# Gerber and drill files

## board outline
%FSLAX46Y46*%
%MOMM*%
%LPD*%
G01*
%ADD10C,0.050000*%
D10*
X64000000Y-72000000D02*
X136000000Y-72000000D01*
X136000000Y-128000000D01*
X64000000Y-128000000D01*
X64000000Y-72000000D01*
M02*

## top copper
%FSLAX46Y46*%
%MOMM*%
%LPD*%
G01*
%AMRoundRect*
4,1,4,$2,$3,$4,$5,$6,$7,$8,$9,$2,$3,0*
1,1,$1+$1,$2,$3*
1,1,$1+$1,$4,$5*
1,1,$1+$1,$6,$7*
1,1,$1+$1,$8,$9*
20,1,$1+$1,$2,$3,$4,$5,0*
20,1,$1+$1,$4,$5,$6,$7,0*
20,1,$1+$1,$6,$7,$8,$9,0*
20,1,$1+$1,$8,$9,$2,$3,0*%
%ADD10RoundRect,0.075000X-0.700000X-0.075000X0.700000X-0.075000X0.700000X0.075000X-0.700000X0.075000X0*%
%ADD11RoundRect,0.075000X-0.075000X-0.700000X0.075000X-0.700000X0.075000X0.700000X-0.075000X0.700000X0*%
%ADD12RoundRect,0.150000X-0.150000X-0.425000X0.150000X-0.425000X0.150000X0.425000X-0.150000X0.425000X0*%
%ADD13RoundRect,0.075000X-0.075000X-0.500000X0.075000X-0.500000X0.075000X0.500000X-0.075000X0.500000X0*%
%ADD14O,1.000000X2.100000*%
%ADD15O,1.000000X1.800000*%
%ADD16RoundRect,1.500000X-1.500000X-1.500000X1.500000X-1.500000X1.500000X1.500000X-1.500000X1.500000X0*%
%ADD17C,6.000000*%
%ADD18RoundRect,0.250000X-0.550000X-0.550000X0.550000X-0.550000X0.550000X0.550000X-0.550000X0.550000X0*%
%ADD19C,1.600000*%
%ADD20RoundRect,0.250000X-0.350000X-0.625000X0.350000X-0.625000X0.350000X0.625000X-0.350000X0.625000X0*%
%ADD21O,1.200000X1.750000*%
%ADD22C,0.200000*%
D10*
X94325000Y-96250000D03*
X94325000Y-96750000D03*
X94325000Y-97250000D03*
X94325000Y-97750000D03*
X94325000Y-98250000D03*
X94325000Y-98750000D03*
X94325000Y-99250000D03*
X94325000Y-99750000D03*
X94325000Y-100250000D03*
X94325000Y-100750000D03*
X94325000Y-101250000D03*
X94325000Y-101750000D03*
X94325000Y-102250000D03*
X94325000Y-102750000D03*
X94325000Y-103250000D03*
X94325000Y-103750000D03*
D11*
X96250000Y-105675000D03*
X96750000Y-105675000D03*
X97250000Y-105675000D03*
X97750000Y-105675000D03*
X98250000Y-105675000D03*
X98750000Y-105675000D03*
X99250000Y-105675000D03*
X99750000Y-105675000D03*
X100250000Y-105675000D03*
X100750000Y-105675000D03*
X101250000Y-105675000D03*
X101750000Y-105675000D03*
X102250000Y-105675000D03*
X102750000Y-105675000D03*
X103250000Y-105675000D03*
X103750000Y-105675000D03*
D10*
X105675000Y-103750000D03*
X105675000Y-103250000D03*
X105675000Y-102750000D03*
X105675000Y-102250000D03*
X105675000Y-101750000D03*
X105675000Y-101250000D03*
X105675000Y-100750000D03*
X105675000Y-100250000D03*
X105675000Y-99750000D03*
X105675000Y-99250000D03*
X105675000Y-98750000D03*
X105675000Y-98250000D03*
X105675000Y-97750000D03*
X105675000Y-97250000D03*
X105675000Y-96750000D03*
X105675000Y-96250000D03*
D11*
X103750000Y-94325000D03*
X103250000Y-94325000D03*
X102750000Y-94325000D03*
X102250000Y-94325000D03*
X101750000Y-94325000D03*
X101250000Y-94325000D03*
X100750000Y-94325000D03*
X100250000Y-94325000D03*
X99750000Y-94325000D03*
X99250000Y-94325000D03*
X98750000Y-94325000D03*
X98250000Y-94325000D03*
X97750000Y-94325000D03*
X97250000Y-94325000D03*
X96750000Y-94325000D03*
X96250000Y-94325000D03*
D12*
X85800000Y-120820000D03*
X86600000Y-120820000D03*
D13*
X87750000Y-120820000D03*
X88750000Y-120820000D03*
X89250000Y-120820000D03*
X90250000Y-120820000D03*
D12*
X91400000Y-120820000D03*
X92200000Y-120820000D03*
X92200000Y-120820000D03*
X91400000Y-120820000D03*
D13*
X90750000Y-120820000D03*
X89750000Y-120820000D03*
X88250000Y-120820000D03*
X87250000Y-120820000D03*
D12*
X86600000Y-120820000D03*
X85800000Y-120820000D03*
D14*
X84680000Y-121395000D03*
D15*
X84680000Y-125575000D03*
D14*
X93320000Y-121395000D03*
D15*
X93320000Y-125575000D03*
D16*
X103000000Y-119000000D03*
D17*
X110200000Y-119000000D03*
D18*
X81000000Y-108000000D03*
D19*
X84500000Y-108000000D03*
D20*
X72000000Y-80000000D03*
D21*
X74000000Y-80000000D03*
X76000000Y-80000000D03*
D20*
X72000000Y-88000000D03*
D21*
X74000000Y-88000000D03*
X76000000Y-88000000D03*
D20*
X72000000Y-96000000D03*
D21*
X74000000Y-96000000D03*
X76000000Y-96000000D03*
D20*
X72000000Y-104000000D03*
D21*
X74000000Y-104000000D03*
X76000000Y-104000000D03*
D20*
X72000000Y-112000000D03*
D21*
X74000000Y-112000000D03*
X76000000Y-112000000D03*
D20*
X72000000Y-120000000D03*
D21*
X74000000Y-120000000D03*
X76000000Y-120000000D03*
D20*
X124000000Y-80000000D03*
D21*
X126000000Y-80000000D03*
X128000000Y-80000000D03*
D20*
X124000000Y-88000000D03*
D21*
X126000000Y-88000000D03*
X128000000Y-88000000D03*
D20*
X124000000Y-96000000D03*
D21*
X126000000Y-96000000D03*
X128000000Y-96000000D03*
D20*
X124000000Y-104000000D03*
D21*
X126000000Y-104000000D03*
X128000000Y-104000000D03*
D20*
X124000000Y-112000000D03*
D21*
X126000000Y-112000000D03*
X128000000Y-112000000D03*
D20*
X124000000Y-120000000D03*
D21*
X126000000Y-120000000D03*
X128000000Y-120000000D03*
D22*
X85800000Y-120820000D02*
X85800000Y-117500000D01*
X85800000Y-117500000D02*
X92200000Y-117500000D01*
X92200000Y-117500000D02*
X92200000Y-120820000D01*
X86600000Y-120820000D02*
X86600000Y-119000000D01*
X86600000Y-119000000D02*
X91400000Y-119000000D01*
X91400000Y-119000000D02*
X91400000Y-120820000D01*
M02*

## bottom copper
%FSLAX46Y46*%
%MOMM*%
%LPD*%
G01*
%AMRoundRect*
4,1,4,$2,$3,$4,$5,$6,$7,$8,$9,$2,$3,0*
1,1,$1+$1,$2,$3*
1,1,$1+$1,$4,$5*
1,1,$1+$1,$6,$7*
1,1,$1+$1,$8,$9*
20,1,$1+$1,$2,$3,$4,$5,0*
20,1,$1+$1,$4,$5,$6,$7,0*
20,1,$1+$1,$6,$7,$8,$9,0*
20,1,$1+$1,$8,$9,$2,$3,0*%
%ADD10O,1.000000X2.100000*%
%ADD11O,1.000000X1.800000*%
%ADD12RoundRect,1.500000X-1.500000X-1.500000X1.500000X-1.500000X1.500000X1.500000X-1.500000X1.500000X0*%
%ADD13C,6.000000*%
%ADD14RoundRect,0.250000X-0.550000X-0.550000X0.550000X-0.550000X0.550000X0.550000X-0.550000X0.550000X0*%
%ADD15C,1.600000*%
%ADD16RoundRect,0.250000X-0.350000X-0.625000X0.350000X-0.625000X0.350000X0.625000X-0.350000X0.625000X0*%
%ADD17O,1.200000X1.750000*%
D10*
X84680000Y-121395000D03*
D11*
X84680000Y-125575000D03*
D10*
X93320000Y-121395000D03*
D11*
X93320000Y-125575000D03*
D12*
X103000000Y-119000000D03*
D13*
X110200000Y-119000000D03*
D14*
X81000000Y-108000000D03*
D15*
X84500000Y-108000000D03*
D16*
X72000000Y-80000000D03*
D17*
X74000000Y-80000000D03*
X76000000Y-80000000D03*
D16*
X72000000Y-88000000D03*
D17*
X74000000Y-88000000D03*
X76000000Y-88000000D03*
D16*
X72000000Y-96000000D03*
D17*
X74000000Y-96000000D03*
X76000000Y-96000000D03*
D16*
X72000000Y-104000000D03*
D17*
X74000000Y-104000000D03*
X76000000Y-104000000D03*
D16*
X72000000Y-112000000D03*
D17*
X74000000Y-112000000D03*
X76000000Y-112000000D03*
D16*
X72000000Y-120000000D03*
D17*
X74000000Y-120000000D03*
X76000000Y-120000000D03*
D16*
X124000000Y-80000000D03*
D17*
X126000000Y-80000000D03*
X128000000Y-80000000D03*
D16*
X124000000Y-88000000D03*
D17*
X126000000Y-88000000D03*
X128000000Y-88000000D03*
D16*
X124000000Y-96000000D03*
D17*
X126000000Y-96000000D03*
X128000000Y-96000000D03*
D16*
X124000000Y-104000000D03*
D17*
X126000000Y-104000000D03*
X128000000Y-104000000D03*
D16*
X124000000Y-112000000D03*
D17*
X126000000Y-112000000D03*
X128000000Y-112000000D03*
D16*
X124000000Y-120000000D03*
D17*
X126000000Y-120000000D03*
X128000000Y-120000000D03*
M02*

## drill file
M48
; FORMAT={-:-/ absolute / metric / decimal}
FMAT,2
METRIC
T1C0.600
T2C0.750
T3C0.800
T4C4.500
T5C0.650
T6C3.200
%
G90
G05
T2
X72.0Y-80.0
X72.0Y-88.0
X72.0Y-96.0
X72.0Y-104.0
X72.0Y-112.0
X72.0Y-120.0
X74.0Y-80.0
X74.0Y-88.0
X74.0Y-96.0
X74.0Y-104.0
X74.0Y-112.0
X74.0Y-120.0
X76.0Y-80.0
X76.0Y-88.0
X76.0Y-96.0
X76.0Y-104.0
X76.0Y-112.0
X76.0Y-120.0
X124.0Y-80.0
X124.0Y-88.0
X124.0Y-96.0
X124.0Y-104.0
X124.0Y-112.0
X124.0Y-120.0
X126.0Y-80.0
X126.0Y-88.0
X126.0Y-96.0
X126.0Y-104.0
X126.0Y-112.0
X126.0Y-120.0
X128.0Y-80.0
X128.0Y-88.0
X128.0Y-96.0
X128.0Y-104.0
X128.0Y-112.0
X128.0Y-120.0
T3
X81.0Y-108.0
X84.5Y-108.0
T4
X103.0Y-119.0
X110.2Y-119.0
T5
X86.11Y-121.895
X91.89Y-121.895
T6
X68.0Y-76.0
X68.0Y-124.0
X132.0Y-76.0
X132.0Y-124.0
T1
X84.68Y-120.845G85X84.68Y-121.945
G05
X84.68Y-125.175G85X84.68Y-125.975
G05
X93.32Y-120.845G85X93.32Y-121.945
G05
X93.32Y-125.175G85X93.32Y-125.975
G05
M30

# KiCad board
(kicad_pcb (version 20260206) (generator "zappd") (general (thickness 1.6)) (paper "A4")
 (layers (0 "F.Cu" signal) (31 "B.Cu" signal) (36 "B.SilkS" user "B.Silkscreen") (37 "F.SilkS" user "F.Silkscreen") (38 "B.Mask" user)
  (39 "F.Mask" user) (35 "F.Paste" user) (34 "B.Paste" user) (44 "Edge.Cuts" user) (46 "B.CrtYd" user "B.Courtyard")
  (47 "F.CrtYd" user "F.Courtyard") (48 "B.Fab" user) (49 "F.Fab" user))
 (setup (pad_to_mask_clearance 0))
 (gr_rect (start 64.0 72.0) (end 136.0 128.0) (stroke (width 0.05) (type default)) (fill none) (layer "Edge.Cuts"))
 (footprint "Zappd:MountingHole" (layer "F.Cu") (at 68.0 76.0)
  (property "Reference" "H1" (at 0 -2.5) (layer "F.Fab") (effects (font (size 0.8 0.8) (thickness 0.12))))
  (pad "" np_thru_hole circle (at 0 0) (size 3.2 3.2) (drill 3.2) (layers "*.Cu" "*.Mask")))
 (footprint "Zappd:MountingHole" (layer "F.Cu") (at 132.0 76.0)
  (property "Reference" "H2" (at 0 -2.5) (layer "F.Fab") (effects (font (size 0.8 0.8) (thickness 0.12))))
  (pad "" np_thru_hole circle (at 0 0) (size 3.2 3.2) (drill 3.2) (layers "*.Cu" "*.Mask")))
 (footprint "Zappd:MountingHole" (layer "F.Cu") (at 132.0 124.0)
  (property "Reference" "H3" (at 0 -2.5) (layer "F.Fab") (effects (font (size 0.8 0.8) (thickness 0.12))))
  (pad "" np_thru_hole circle (at 0 0) (size 3.2 3.2) (drill 3.2) (layers "*.Cu" "*.Mask")))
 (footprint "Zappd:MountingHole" (layer "F.Cu") (at 68.0 124.0)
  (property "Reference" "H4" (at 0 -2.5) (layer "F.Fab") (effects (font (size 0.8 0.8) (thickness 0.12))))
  (pad "" np_thru_hole circle (at 0 0) (size 3.2 3.2) (drill 3.2) (layers "*.Cu" "*.Mask")))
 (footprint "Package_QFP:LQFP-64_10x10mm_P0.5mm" (layer "F.Cu") (at 100 100)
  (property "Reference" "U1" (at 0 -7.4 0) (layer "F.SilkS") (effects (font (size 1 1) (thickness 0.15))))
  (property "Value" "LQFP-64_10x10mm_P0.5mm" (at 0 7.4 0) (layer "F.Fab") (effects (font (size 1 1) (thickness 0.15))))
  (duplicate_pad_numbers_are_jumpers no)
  (pad "1" smd roundrect (at -5.675 -3.75) (size 1.55 0.3) (layers "F.Cu" "F.Mask" "F.Paste") (roundrect_rratio 0.25))
  (pad "2" smd roundrect (at -5.675 -3.25) (size 1.55 0.3) (layers "F.Cu" "F.Mask" "F.Paste") (roundrect_rratio 0.25))
  (pad "3" smd roundrect (at -5.675 -2.75) (size 1.55 0.3) (layers "F.Cu" "F.Mask" "F.Paste") (roundrect_rratio 0.25))
  (pad "4" smd roundrect (at -5.675 -2.25) (size 1.55 0.3) (layers "F.Cu" "F.Mask" "F.Paste") (roundrect_rratio 0.25))
  (pad "5" smd roundrect (at -5.675 -1.75) (size 1.55 0.3) (layers "F.Cu" "F.Mask" "F.Paste") (roundrect_rratio 0.25))
  (pad "6" smd roundrect (at -5.675 -1.25) (size 1.55 0.3) (layers "F.Cu" "F.Mask" "F.Paste") (roundrect_rratio 0.25))
  (pad "7" smd roundrect (at -5.675 -0.75) (size 1.55 0.3) (layers "F.Cu" "F.Mask" "F.Paste") (roundrect_rratio 0.25))
  (pad "8" smd roundrect (at -5.675 -0.25) (size 1.55 0.3) (layers "F.Cu" "F.Mask" "F.Paste") (roundrect_rratio 0.25))
  (pad "9" smd roundrect (at -5.675 0.25) (size 1.55 0.3) (layers "F.Cu" "F.Mask" "F.Paste") (roundrect_rratio 0.25))
  (pad "10" smd roundrect (at -5.675 0.75) (size 1.55 0.3) (layers "F.Cu" "F.Mask" "F.Paste") (roundrect_rratio 0.25))
  (pad "11" smd roundrect (at -5.675 1.25) (size 1.55 0.3) (layers "F.Cu" "F.Mask" "F.Paste") (roundrect_rratio 0.25))
  (pad "12" smd roundrect (at -5.675 1.75) (size 1.55 0.3) (layers "F.Cu" "F.Mask" "F.Paste") (roundrect_rratio 0.25))
  (pad "13" smd roundrect (at -5.675 2.25) (size 1.55 0.3) (layers "F.Cu" "F.Mask" "F.Paste") (roundrect_rratio 0.25))
  (pad "14" smd roundrect (at -5.675 2.75) (size 1.55 0.3) (layers "F.Cu" "F.Mask" "F.Paste") (roundrect_rratio 0.25))
  (pad "15" smd roundrect (at -5.675 3.25) (size 1.55 0.3) (layers "F.Cu" "F.Mask" "F.Paste") (roundrect_rratio 0.25))
  (pad "16" smd roundrect (at -5.675 3.75) (size 1.55 0.3) (layers "F.Cu" "F.Mask" "F.Paste") (roundrect_rratio 0.25))
  (pad "17" smd roundrect (at -3.75 5.675) (size 0.3 1.55) (layers "F.Cu" "F.Mask" "F.Paste") (roundrect_rratio 0.25))
  (pad "18" smd roundrect (at -3.25 5.675) (size 0.3 1.55) (layers "F.Cu" "F.Mask" "F.Paste") (roundrect_rratio 0.25))
  (pad "19" smd roundrect (at -2.75 5.675) (size 0.3 1.55) (layers "F.Cu" "F.Mask" "F.Paste") (roundrect_rratio 0.25))
  (pad "20" smd roundrect (at -2.25 5.675) (size 0.3 1.55) (layers "F.Cu" "F.Mask" "F.Paste") (roundrect_rratio 0.25))
  (pad "21" smd roundrect (at -1.75 5.675) (size 0.3 1.55) (layers "F.Cu" "F.Mask" "F.Paste") (roundrect_rratio 0.25))
  (pad "22" smd roundrect (at -1.25 5.675) (size 0.3 1.55) (layers "F.Cu" "F.Mask" "F.Paste") (roundrect_rratio 0.25))
  (pad "23" smd roundrect (at -0.75 5.675) (size 0.3 1.55) (layers "F.Cu" "F.Mask" "F.Paste") (roundrect_rratio 0.25))
  (pad "24" smd roundrect (at -0.25 5.675) (size 0.3 1.55) (layers "F.Cu" "F.Mask" "F.Paste") (roundrect_rratio 0.25))
  (pad "25" smd roundrect (at 0.25 5.675) (size 0.3 1.55) (layers "F.Cu" "F.Mask" "F.Paste") (roundrect_rratio 0.25))
  (pad "26" smd roundrect (at 0.75 5.675) (size 0.3 1.55) (layers "F.Cu" "F.Mask" "F.Paste") (roundrect_rratio 0.25))
  (pad "27" smd roundrect (at 1.25 5.675) (size 0.3 1.55) (layers "F.Cu" "F.Mask" "F.Paste") (roundrect_rratio 0.25))
  (pad "28" smd roundrect (at 1.75 5.675) (size 0.3 1.55) (layers "F.Cu" "F.Mask" "F.Paste") (roundrect_rratio 0.25))
  (pad "29" smd roundrect (at 2.25 5.675) (size 0.3 1.55) (layers "F.Cu" "F.Mask" "F.Paste") (roundrect_rratio 0.25))
  (pad "30" smd roundrect (at 2.75 5.675) (size 0.3 1.55) (layers "F.Cu" "F.Mask" "F.Paste") (roundrect_rratio 0.25))
  (pad "31" smd roundrect (at 3.25 5.675) (size 0.3 1.55) (layers "F.Cu" "F.Mask" "F.Paste") (roundrect_rratio 0.25))
  (pad "32" smd roundrect (at 3.75 5.675) (size 0.3 1.55) (layers "F.Cu" "F.Mask" "F.Paste") (roundrect_rratio 0.25))
  (pad "33" smd roundrect (at 5.675 3.75) (size 1.55 0.3) (layers "F.Cu" "F.Mask" "F.Paste") (roundrect_rratio 0.25))
  (pad "34" smd roundrect (at 5.675 3.25) (size 1.55 0.3) (layers "F.Cu" "F.Mask" "F.Paste") (roundrect_rratio 0.25))
  (pad "35" smd roundrect (at 5.675 2.75) (size 1.55 0.3) (layers "F.Cu" "F.Mask" "F.Paste") (roundrect_rratio 0.25))
  (pad "36" smd roundrect (at 5.675 2.25) (size 1.55 0.3) (layers "F.Cu" "F.Mask" "F.Paste") (roundrect_rratio 0.25))
  (pad "37" smd roundrect (at 5.675 1.75) (size 1.55 0.3) (layers "F.Cu" "F.Mask" "F.Paste") (roundrect_rratio 0.25))
  (pad "38" smd roundrect (at 5.675 1.25) (size 1.55 0.3) (layers "F.Cu" "F.Mask" "F.Paste") (roundrect_rratio 0.25))
  (pad "39" smd roundrect (at 5.675 0.75) (size 1.55 0.3) (layers "F.Cu" "F.Mask" "F.Paste") (roundrect_rratio 0.25))
  (pad "40" smd roundrect (at 5.675 0.25) (size 1.55 0.3) (layers "F.Cu" "F.Mask" "F.Paste") (roundrect_rratio 0.25))
  (pad "41" smd roundrect (at 5.675 -0.25) (size 1.55 0.3) (layers "F.Cu" "F.Mask" "F.Paste") (roundrect_rratio 0.25))
  (pad "42" smd roundrect (at 5.675 -0.75) (size 1.55 0.3) (layers "F.Cu" "F.Mask" "F.Paste") (roundrect_rratio 0.25))
  (pad "43" smd roundrect (at 5.675 -1.25) (size 1.55 0.3) (layers "F.Cu" "F.Mask" "F.Paste") (roundrect_rratio 0.25))
  (pad "44" smd roundrect (at 5.675 -1.75) (size 1.55 0.3) (layers "F.Cu" "F.Mask" "F.Paste") (roundrect_rratio 0.25))
  (pad "45" smd roundrect (at 5.675 -2.25) (size 1.55 0.3) (layers "F.Cu" "F.Mask" "F.Paste") (roundrect_rratio 0.25))
  (pad "46" smd roundrect (at 5.675 -2.75) (size 1.55 0.3) (layers "F.Cu" "F.Mask" "F.Paste") (roundrect_rratio 0.25))
  (pad "47" smd roundrect (at 5.675 -3.25) (size 1.55 0.3) (layers "F.Cu" "F.Mask" "F.Paste") (roundrect_rratio 0.25))
  (pad "48" smd roundrect (at 5.675 -3.75) (size 1.55 0.3) (layers "F.Cu" "F.Mask" "F.Paste") (roundrect_rratio 0.25))
  (pad "49" smd roundrect (at 3.75 -5.675) (size 0.3 1.55) (layers "F.Cu" "F.Mask" "F.Paste") (roundrect_rratio 0.25))
  (pad "50" smd roundrect (at 3.25 -5.675) (size 0.3 1.55) (layers "F.Cu" "F.Mask" "F.Paste") (roundrect_rratio 0.25))
  (pad "51" smd roundrect (at 2.75 -5.675) (size 0.3 1.55) (layers "F.Cu" "F.Mask" "F.Paste") (roundrect_rratio 0.25))
  (pad "52" smd roundrect (at 2.25 -5.675) (size 0.3 1.55) (layers "F.Cu" "F.Mask" "F.Paste") (roundrect_rratio 0.25))
  (pad "53" smd roundrect (at 1.75 -5.675) (size 0.3 1.55) (layers "F.Cu" "F.Mask" "F.Paste") (roundrect_rratio 0.25))
  (pad "54" smd roundrect (at 1.25 -5.675) (size 0.3 1.55) (layers "F.Cu" "F.Mask" "F.Paste") (roundrect_rratio 0.25))
  (pad "55" smd roundrect (at 0.75 -5.675) (size 0.3 1.55) (layers "F.Cu" "F.Mask" "F.Paste") (roundrect_rratio 0.25))
  (pad "56" smd roundrect (at 0.25 -5.675) (size 0.3 1.55) (layers "F.Cu" "F.Mask" "F.Paste") (roundrect_rratio 0.25))
  (pad "57" smd roundrect (at -0.25 -5.675) (size 0.3 1.55) (layers "F.Cu" "F.Mask" "F.Paste") (roundrect_rratio 0.25))
  (pad "58" smd roundrect (at -0.75 -5.675) (size 0.3 1.55) (layers "F.Cu" "F.Mask" "F.Paste") (roundrect_rratio 0.25))
  (pad "59" smd roundrect (at -1.25 -5.675) (size 0.3 1.55) (layers "F.Cu" "F.Mask" "F.Paste") (roundrect_rratio 0.25))
  (pad "60" smd roundrect (at -1.75 -5.675) (size 0.3 1.55) (layers "F.Cu" "F.Mask" "F.Paste") (roundrect_rratio 0.25))
  (pad "61" smd roundrect (at -2.25 -5.675) (size 0.3 1.55) (layers "F.Cu" "F.Mask" "F.Paste") (roundrect_rratio 0.25))
  (pad "62" smd roundrect (at -2.75 -5.675) (size 0.3 1.55) (layers "F.Cu" "F.Mask" "F.Paste") (roundrect_rratio 0.25))
  (pad "63" smd roundrect (at -3.25 -5.675) (size 0.3 1.55) (layers "F.Cu" "F.Mask" "F.Paste") (roundrect_rratio 0.25))
  (pad "64" smd roundrect (at -3.75 -5.675) (size 0.3 1.55) (layers "F.Cu" "F.Mask" "F.Paste") (roundrect_rratio 0.25)))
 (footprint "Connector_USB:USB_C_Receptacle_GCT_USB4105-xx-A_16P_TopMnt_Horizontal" (layer "F.Cu") (at 89 124.5)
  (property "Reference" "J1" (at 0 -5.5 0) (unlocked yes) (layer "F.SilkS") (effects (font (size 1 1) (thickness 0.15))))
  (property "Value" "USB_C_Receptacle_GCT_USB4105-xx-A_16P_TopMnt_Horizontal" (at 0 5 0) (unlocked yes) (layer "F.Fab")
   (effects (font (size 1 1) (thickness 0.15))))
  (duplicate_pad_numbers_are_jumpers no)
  (pad "" np_thru_hole circle (at -2.89 -2.605) (size 0.65 0.65) (drill 0.65) (layers "*.Cu" "*.Mask"))
  (pad "" np_thru_hole circle (at 2.89 -2.605) (size 0.65 0.65) (drill 0.65) (layers "*.Cu" "*.Mask"))
  (pad "A1" smd roundrect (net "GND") (at -3.2 -3.68) (size 0.6 1.15) (layers "F.Cu" "F.Mask" "F.Paste") (roundrect_rratio 0.25))
  (pad "A4" smd roundrect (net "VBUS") (at -2.4 -3.68) (size 0.6 1.15) (layers "F.Cu" "F.Mask" "F.Paste") (roundrect_rratio 0.25))
  (pad "A5" smd roundrect (at -1.25 -3.68) (size 0.3 1.15) (layers "F.Cu" "F.Mask" "F.Paste") (roundrect_rratio 0.25))
  (pad "A6" smd roundrect (at -0.25 -3.68) (size 0.3 1.15) (layers "F.Cu" "F.Mask" "F.Paste") (roundrect_rratio 0.25))
  (pad "A7" smd roundrect (at 0.25 -3.68) (size 0.3 1.15) (layers "F.Cu" "F.Mask" "F.Paste") (roundrect_rratio 0.25))
  (pad "A8" smd roundrect (at 1.25 -3.68) (size 0.3 1.15) (layers "F.Cu" "F.Mask" "F.Paste") (roundrect_rratio 0.25))
  (pad "A9" smd roundrect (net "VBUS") (at 2.4 -3.68) (size 0.6 1.15) (layers "F.Cu" "F.Mask" "F.Paste") (roundrect_rratio 0.25))
  (pad "A12" smd roundrect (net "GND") (at 3.2 -3.68) (size 0.6 1.15) (layers "F.Cu" "F.Mask" "F.Paste") (roundrect_rratio 0.25))
  (pad "B1" smd roundrect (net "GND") (at 3.2 -3.68) (size 0.6 1.15) (layers "F.Cu" "F.Mask" "F.Paste") (roundrect_rratio 0.25))
  (pad "B4" smd roundrect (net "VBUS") (at 2.4 -3.68) (size 0.6 1.15) (layers "F.Cu" "F.Mask" "F.Paste") (roundrect_rratio 0.25))
  (pad "B5" smd roundrect (at 1.75 -3.68) (size 0.3 1.15) (layers "F.Cu" "F.Mask" "F.Paste") (roundrect_rratio 0.25))
  (pad "B6" smd roundrect (at 0.75 -3.68) (size 0.3 1.15) (layers "F.Cu" "F.Mask" "F.Paste") (roundrect_rratio 0.25))
  (pad "B7" smd roundrect (at -0.75 -3.68) (size 0.3 1.15) (layers "F.Cu" "F.Mask" "F.Paste") (roundrect_rratio 0.25))
  (pad "B8" smd roundrect (at -1.75 -3.68) (size 0.3 1.15) (layers "F.Cu" "F.Mask" "F.Paste") (roundrect_rratio 0.25))
  (pad "B9" smd roundrect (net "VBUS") (at -2.4 -3.68) (size 0.6 1.15) (layers "F.Cu" "F.Mask" "F.Paste") (roundrect_rratio 0.25))
  (pad "B12" smd roundrect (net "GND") (at -3.2 -3.68) (size 0.6 1.15) (layers "F.Cu" "F.Mask" "F.Paste") (roundrect_rratio 0.25))
  (pad "SH" thru_hole oval (at -4.32 -3.105) (size 1 2.1) (drill oval 0.6 1.7) (layers "*.Cu" "*.Mask" "F.Paste") (remove_unused_layers no))
  (pad "SH" thru_hole oval (at -4.32 1.075) (size 1 1.8) (drill oval 0.6 1.4) (layers "*.Cu" "*.Mask" "F.Paste") (remove_unused_layers no))
  (pad "SH" thru_hole oval (at 4.32 -3.105) (size 1 2.1) (drill oval 0.6 1.7) (layers "*.Cu" "*.Mask" "F.Paste") (remove_unused_layers no))
  (pad "SH" thru_hole oval (at 4.32 1.075) (size 1 1.8) (drill oval 0.6 1.4) (layers "*.Cu" "*.Mask" "F.Paste") (remove_unused_layers no)))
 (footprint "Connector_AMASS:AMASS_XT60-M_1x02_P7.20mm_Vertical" (layer "F.Cu") (at 103 119)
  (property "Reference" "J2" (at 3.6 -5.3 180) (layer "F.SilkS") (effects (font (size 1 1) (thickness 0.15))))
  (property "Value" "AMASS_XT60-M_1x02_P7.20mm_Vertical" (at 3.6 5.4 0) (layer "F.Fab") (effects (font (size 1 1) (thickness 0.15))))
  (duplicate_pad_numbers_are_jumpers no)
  (pad "1" thru_hole roundrect (at 0 0) (size 6 6) (drill 4.5) (layers "*.Cu" "*.Mask") (remove_unused_layers no) (roundrect_rratio 0.25))
  (pad "2" thru_hole circle (at 7.2 0) (size 6 6) (drill 4.5) (layers "*.Cu" "*.Mask") (remove_unused_layers no)))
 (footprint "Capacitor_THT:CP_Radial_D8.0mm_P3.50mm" (layer "F.Cu") (at 81 108)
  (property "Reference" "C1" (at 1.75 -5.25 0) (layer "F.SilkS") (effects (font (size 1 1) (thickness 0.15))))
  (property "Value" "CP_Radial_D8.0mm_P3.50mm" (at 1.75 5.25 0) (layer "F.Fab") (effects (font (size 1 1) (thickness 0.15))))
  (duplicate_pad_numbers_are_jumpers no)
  (pad "1" thru_hole roundrect (at 0 0) (size 1.6 1.6) (drill 0.8) (layers "*.Cu" "*.Mask") (remove_unused_layers no)
   (roundrect_rratio 0.15625))
  (pad "2" thru_hole circle (at 3.5 0) (size 1.6 1.6) (drill 0.8) (layers "*.Cu" "*.Mask") (remove_unused_layers no)))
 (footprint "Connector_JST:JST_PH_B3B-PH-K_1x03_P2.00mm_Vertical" (layer "F.Cu") (at 72 80)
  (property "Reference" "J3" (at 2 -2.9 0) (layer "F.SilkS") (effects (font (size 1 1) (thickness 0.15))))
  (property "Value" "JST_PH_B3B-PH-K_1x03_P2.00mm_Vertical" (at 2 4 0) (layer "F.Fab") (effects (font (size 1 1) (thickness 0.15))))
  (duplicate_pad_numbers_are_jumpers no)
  (pad "1" thru_hole roundrect (at 0 0) (size 1.2 1.75) (drill 0.75) (layers "*.Cu" "*.Mask") (remove_unused_layers no)
   (roundrect_rratio 0.208333))
  (pad "2" thru_hole oval (at 2 0) (size 1.2 1.75) (drill 0.75) (layers "*.Cu" "*.Mask") (remove_unused_layers no))
  (pad "3" thru_hole oval (at 4 0) (size 1.2 1.75) (drill 0.75) (layers "*.Cu" "*.Mask") (remove_unused_layers no)))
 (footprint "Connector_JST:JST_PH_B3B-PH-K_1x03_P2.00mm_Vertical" (layer "F.Cu") (at 72 88)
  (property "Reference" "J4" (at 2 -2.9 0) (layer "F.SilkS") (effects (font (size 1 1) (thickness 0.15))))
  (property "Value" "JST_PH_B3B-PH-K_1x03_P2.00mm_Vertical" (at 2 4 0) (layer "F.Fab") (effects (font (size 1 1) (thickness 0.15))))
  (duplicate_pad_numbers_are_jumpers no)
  (pad "1" thru_hole roundrect (at 0 0) (size 1.2 1.75) (drill 0.75) (layers "*.Cu" "*.Mask") (remove_unused_layers no)
   (roundrect_rratio 0.208333))
  (pad "2" thru_hole oval (at 2 0) (size 1.2 1.75) (drill 0.75) (layers "*.Cu" "*.Mask") (remove_unused_layers no))
  (pad "3" thru_hole oval (at 4 0) (size 1.2 1.75) (drill 0.75) (layers "*.Cu" "*.Mask") (remove_unused_layers no)))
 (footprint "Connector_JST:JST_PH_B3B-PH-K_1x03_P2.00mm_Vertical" (layer "F.Cu") (at 72 96)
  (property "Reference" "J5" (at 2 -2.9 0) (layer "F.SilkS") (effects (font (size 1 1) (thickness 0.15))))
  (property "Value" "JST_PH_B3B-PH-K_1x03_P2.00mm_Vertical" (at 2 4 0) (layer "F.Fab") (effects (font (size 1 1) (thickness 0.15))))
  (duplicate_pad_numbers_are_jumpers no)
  (pad "1" thru_hole roundrect (at 0 0) (size 1.2 1.75) (drill 0.75) (layers "*.Cu" "*.Mask") (remove_unused_layers no)
   (roundrect_rratio 0.208333))
  (pad "2" thru_hole oval (at 2 0) (size 1.2 1.75) (drill 0.75) (layers "*.Cu" "*.Mask") (remove_unused_layers no))
  (pad "3" thru_hole oval (at 4 0) (size 1.2 1.75) (drill 0.75) (layers "*.Cu" "*.Mask") (remove_unused_layers no)))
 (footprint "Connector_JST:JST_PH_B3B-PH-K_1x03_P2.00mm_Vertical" (layer "F.Cu") (at 72 104)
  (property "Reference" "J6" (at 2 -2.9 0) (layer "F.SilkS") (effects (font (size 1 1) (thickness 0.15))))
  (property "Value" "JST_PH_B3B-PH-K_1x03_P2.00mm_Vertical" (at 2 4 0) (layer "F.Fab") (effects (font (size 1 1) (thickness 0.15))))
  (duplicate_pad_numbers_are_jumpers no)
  (pad "1" thru_hole roundrect (at 0 0) (size 1.2 1.75) (drill 0.75) (layers "*.Cu" "*.Mask") (remove_unused_layers no)
   (roundrect_rratio 0.208333))
  (pad "2" thru_hole oval (at 2 0) (size 1.2 1.75) (drill 0.75) (layers "*.Cu" "*.Mask") (remove_unused_layers no))
  (pad "3" thru_hole oval (at 4 0) (size 1.2 1.75) (drill 0.75) (layers "*.Cu" "*.Mask") (remove_unused_layers no)))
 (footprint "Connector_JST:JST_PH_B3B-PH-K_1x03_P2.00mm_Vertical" (layer "F.Cu") (at 72 112)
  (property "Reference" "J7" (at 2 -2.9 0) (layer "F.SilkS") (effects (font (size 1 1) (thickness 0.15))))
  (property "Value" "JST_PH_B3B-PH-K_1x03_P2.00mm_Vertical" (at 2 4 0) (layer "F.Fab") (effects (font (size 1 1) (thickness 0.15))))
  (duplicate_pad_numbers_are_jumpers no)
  (pad "1" thru_hole roundrect (at 0 0) (size 1.2 1.75) (drill 0.75) (layers "*.Cu" "*.Mask") (remove_unused_layers no)
   (roundrect_rratio 0.208333))
  (pad "2" thru_hole oval (at 2 0) (size 1.2 1.75) (drill 0.75) (layers "*.Cu" "*.Mask") (remove_unused_layers no))
  (pad "3" thru_hole oval (at 4 0) (size 1.2 1.75) (drill 0.75) (layers "*.Cu" "*.Mask") (remove_unused_layers no)))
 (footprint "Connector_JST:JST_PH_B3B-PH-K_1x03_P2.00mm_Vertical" (layer "F.Cu") (at 72 120)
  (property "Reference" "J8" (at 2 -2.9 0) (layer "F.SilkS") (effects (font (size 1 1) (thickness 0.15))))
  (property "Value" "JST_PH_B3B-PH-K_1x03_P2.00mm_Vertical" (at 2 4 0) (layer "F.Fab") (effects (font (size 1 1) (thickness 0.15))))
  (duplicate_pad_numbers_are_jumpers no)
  (pad "1" thru_hole roundrect (at 0 0) (size 1.2 1.75) (drill 0.75) (layers "*.Cu" "*.Mask") (remove_unused_layers no)
   (roundrect_rratio 0.208333))
  (pad "2" thru_hole oval (at 2 0) (size 1.2 1.75) (drill 0.75) (layers "*.Cu" "*.Mask") (remove_unused_layers no))
  (pad "3" thru_hole oval (at 4 0) (size 1.2 1.75) (drill 0.75) (layers "*.Cu" "*.Mask") (remove_unused_layers no)))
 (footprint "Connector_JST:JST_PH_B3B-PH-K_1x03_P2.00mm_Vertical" (layer "F.Cu") (at 124 80)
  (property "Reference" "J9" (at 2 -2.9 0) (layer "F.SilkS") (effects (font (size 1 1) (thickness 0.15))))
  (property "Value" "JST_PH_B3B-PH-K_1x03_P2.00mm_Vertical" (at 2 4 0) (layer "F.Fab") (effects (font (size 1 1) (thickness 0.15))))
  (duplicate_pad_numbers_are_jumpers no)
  (pad "1" thru_hole roundrect (at 0 0) (size 1.2 1.75) (drill 0.75) (layers "*.Cu" "*.Mask") (remove_unused_layers no)
   (roundrect_rratio 0.208333))
  (pad "2" thru_hole oval (at 2 0) (size 1.2 1.75) (drill 0.75) (layers "*.Cu" "*.Mask") (remove_unused_layers no))
  (pad "3" thru_hole oval (at 4 0) (size 1.2 1.75) (drill 0.75) (layers "*.Cu" "*.Mask") (remove_unused_layers no)))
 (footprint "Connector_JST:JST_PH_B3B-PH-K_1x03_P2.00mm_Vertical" (layer "F.Cu") (at 124 88)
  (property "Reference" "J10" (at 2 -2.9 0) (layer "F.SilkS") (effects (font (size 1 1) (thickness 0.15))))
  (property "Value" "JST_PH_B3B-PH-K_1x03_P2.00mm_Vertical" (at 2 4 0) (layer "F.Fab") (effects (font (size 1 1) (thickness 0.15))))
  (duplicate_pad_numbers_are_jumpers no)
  (pad "1" thru_hole roundrect (at 0 0) (size 1.2 1.75) (drill 0.75) (layers "*.Cu" "*.Mask") (remove_unused_layers no)
   (roundrect_rratio 0.208333))
  (pad "2" thru_hole oval (at 2 0) (size 1.2 1.75) (drill 0.75) (layers "*.Cu" "*.Mask") (remove_unused_layers no))
  (pad "3" thru_hole oval (at 4 0) (size 1.2 1.75) (drill 0.75) (layers "*.Cu" "*.Mask") (remove_unused_layers no)))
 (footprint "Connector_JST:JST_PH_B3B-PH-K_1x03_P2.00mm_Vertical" (layer "F.Cu") (at 124 96)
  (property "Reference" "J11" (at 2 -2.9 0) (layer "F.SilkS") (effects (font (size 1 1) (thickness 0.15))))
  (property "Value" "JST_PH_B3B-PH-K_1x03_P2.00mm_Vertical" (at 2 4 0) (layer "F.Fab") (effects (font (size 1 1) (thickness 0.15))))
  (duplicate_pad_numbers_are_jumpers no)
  (pad "1" thru_hole roundrect (at 0 0) (size 1.2 1.75) (drill 0.75) (layers "*.Cu" "*.Mask") (remove_unused_layers no)
   (roundrect_rratio 0.208333))
  (pad "2" thru_hole oval (at 2 0) (size 1.2 1.75) (drill 0.75) (layers "*.Cu" "*.Mask") (remove_unused_layers no))
  (pad "3" thru_hole oval (at 4 0) (size 1.2 1.75) (drill 0.75) (layers "*.Cu" "*.Mask") (remove_unused_layers no)))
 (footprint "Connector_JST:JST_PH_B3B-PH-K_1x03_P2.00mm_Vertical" (layer "F.Cu") (at 124 104)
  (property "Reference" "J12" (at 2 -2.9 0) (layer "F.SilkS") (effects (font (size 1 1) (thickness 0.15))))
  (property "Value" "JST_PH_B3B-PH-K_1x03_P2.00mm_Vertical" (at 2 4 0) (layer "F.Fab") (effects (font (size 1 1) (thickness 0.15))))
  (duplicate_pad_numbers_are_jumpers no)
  (pad "1" thru_hole roundrect (at 0 0) (size 1.2 1.75) (drill 0.75) (layers "*.Cu" "*.Mask") (remove_unused_layers no)
   (roundrect_rratio 0.208333))
  (pad "2" thru_hole oval (at 2 0) (size 1.2 1.75) (drill 0.75) (layers "*.Cu" "*.Mask") (remove_unused_layers no))
  (pad "3" thru_hole oval (at 4 0) (size 1.2 1.75) (drill 0.75) (layers "*.Cu" "*.Mask") (remove_unused_layers no)))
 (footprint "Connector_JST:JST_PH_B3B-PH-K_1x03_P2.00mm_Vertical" (layer "F.Cu") (at 124 112)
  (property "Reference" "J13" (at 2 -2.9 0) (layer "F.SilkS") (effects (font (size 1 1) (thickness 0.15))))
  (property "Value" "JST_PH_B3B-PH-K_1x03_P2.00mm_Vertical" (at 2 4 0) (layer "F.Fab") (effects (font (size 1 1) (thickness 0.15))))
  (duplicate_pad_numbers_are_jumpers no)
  (pad "1" thru_hole roundrect (at 0 0) (size 1.2 1.75) (drill 0.75) (layers "*.Cu" "*.Mask") (remove_unused_layers no)
   (roundrect_rratio 0.208333))
  (pad "2" thru_hole oval (at 2 0) (size 1.2 1.75) (drill 0.75) (layers "*.Cu" "*.Mask") (remove_unused_layers no))
  (pad "3" thru_hole oval (at 4 0) (size 1.2 1.75) (drill 0.75) (layers "*.Cu" "*.Mask") (remove_unused_layers no)))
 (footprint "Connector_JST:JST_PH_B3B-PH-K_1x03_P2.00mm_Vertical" (layer "F.Cu") (at 124 120)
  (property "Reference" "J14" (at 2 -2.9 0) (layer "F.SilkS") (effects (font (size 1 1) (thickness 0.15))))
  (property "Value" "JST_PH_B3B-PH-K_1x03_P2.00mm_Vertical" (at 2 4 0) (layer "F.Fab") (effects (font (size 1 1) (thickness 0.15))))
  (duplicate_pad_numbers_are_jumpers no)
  (pad "1" thru_hole roundrect (at 0 0) (size 1.2 1.75) (drill 0.75) (layers "*.Cu" "*.Mask") (remove_unused_layers no)
   (roundrect_rratio 0.208333))
  (pad "2" thru_hole oval (at 2 0) (size 1.2 1.75) (drill 0.75) (layers "*.Cu" "*.Mask") (remove_unused_layers no))
  (pad "3" thru_hole oval (at 4 0) (size 1.2 1.75) (drill 0.75) (layers "*.Cu" "*.Mask") (remove_unused_layers no)))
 (segment (start 85.8000 120.8200) (end 85.8000 117.5000) (width 0.2) (layer "F.Cu") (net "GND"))
 (segment (start 85.8000 117.5000) (end 92.2000 117.5000) (width 0.2) (layer "F.Cu") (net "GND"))
 (segment (start 92.2000 117.5000) (end 92.2000 120.8200) (width 0.2) (layer "F.Cu") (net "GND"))
 (segment (start 86.6000 120.8200) (end 86.6000 119.0000) (width 0.2) (layer "F.Cu") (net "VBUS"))
 (segment (start 86.6000 119.0000) (end 91.4000 119.0000) (width 0.2) (layer "F.Cu") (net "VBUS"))
 (segment (start 91.4000 119.0000) (end 91.4000 120.8200) (width 0.2) (layer "F.Cu") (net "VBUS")))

